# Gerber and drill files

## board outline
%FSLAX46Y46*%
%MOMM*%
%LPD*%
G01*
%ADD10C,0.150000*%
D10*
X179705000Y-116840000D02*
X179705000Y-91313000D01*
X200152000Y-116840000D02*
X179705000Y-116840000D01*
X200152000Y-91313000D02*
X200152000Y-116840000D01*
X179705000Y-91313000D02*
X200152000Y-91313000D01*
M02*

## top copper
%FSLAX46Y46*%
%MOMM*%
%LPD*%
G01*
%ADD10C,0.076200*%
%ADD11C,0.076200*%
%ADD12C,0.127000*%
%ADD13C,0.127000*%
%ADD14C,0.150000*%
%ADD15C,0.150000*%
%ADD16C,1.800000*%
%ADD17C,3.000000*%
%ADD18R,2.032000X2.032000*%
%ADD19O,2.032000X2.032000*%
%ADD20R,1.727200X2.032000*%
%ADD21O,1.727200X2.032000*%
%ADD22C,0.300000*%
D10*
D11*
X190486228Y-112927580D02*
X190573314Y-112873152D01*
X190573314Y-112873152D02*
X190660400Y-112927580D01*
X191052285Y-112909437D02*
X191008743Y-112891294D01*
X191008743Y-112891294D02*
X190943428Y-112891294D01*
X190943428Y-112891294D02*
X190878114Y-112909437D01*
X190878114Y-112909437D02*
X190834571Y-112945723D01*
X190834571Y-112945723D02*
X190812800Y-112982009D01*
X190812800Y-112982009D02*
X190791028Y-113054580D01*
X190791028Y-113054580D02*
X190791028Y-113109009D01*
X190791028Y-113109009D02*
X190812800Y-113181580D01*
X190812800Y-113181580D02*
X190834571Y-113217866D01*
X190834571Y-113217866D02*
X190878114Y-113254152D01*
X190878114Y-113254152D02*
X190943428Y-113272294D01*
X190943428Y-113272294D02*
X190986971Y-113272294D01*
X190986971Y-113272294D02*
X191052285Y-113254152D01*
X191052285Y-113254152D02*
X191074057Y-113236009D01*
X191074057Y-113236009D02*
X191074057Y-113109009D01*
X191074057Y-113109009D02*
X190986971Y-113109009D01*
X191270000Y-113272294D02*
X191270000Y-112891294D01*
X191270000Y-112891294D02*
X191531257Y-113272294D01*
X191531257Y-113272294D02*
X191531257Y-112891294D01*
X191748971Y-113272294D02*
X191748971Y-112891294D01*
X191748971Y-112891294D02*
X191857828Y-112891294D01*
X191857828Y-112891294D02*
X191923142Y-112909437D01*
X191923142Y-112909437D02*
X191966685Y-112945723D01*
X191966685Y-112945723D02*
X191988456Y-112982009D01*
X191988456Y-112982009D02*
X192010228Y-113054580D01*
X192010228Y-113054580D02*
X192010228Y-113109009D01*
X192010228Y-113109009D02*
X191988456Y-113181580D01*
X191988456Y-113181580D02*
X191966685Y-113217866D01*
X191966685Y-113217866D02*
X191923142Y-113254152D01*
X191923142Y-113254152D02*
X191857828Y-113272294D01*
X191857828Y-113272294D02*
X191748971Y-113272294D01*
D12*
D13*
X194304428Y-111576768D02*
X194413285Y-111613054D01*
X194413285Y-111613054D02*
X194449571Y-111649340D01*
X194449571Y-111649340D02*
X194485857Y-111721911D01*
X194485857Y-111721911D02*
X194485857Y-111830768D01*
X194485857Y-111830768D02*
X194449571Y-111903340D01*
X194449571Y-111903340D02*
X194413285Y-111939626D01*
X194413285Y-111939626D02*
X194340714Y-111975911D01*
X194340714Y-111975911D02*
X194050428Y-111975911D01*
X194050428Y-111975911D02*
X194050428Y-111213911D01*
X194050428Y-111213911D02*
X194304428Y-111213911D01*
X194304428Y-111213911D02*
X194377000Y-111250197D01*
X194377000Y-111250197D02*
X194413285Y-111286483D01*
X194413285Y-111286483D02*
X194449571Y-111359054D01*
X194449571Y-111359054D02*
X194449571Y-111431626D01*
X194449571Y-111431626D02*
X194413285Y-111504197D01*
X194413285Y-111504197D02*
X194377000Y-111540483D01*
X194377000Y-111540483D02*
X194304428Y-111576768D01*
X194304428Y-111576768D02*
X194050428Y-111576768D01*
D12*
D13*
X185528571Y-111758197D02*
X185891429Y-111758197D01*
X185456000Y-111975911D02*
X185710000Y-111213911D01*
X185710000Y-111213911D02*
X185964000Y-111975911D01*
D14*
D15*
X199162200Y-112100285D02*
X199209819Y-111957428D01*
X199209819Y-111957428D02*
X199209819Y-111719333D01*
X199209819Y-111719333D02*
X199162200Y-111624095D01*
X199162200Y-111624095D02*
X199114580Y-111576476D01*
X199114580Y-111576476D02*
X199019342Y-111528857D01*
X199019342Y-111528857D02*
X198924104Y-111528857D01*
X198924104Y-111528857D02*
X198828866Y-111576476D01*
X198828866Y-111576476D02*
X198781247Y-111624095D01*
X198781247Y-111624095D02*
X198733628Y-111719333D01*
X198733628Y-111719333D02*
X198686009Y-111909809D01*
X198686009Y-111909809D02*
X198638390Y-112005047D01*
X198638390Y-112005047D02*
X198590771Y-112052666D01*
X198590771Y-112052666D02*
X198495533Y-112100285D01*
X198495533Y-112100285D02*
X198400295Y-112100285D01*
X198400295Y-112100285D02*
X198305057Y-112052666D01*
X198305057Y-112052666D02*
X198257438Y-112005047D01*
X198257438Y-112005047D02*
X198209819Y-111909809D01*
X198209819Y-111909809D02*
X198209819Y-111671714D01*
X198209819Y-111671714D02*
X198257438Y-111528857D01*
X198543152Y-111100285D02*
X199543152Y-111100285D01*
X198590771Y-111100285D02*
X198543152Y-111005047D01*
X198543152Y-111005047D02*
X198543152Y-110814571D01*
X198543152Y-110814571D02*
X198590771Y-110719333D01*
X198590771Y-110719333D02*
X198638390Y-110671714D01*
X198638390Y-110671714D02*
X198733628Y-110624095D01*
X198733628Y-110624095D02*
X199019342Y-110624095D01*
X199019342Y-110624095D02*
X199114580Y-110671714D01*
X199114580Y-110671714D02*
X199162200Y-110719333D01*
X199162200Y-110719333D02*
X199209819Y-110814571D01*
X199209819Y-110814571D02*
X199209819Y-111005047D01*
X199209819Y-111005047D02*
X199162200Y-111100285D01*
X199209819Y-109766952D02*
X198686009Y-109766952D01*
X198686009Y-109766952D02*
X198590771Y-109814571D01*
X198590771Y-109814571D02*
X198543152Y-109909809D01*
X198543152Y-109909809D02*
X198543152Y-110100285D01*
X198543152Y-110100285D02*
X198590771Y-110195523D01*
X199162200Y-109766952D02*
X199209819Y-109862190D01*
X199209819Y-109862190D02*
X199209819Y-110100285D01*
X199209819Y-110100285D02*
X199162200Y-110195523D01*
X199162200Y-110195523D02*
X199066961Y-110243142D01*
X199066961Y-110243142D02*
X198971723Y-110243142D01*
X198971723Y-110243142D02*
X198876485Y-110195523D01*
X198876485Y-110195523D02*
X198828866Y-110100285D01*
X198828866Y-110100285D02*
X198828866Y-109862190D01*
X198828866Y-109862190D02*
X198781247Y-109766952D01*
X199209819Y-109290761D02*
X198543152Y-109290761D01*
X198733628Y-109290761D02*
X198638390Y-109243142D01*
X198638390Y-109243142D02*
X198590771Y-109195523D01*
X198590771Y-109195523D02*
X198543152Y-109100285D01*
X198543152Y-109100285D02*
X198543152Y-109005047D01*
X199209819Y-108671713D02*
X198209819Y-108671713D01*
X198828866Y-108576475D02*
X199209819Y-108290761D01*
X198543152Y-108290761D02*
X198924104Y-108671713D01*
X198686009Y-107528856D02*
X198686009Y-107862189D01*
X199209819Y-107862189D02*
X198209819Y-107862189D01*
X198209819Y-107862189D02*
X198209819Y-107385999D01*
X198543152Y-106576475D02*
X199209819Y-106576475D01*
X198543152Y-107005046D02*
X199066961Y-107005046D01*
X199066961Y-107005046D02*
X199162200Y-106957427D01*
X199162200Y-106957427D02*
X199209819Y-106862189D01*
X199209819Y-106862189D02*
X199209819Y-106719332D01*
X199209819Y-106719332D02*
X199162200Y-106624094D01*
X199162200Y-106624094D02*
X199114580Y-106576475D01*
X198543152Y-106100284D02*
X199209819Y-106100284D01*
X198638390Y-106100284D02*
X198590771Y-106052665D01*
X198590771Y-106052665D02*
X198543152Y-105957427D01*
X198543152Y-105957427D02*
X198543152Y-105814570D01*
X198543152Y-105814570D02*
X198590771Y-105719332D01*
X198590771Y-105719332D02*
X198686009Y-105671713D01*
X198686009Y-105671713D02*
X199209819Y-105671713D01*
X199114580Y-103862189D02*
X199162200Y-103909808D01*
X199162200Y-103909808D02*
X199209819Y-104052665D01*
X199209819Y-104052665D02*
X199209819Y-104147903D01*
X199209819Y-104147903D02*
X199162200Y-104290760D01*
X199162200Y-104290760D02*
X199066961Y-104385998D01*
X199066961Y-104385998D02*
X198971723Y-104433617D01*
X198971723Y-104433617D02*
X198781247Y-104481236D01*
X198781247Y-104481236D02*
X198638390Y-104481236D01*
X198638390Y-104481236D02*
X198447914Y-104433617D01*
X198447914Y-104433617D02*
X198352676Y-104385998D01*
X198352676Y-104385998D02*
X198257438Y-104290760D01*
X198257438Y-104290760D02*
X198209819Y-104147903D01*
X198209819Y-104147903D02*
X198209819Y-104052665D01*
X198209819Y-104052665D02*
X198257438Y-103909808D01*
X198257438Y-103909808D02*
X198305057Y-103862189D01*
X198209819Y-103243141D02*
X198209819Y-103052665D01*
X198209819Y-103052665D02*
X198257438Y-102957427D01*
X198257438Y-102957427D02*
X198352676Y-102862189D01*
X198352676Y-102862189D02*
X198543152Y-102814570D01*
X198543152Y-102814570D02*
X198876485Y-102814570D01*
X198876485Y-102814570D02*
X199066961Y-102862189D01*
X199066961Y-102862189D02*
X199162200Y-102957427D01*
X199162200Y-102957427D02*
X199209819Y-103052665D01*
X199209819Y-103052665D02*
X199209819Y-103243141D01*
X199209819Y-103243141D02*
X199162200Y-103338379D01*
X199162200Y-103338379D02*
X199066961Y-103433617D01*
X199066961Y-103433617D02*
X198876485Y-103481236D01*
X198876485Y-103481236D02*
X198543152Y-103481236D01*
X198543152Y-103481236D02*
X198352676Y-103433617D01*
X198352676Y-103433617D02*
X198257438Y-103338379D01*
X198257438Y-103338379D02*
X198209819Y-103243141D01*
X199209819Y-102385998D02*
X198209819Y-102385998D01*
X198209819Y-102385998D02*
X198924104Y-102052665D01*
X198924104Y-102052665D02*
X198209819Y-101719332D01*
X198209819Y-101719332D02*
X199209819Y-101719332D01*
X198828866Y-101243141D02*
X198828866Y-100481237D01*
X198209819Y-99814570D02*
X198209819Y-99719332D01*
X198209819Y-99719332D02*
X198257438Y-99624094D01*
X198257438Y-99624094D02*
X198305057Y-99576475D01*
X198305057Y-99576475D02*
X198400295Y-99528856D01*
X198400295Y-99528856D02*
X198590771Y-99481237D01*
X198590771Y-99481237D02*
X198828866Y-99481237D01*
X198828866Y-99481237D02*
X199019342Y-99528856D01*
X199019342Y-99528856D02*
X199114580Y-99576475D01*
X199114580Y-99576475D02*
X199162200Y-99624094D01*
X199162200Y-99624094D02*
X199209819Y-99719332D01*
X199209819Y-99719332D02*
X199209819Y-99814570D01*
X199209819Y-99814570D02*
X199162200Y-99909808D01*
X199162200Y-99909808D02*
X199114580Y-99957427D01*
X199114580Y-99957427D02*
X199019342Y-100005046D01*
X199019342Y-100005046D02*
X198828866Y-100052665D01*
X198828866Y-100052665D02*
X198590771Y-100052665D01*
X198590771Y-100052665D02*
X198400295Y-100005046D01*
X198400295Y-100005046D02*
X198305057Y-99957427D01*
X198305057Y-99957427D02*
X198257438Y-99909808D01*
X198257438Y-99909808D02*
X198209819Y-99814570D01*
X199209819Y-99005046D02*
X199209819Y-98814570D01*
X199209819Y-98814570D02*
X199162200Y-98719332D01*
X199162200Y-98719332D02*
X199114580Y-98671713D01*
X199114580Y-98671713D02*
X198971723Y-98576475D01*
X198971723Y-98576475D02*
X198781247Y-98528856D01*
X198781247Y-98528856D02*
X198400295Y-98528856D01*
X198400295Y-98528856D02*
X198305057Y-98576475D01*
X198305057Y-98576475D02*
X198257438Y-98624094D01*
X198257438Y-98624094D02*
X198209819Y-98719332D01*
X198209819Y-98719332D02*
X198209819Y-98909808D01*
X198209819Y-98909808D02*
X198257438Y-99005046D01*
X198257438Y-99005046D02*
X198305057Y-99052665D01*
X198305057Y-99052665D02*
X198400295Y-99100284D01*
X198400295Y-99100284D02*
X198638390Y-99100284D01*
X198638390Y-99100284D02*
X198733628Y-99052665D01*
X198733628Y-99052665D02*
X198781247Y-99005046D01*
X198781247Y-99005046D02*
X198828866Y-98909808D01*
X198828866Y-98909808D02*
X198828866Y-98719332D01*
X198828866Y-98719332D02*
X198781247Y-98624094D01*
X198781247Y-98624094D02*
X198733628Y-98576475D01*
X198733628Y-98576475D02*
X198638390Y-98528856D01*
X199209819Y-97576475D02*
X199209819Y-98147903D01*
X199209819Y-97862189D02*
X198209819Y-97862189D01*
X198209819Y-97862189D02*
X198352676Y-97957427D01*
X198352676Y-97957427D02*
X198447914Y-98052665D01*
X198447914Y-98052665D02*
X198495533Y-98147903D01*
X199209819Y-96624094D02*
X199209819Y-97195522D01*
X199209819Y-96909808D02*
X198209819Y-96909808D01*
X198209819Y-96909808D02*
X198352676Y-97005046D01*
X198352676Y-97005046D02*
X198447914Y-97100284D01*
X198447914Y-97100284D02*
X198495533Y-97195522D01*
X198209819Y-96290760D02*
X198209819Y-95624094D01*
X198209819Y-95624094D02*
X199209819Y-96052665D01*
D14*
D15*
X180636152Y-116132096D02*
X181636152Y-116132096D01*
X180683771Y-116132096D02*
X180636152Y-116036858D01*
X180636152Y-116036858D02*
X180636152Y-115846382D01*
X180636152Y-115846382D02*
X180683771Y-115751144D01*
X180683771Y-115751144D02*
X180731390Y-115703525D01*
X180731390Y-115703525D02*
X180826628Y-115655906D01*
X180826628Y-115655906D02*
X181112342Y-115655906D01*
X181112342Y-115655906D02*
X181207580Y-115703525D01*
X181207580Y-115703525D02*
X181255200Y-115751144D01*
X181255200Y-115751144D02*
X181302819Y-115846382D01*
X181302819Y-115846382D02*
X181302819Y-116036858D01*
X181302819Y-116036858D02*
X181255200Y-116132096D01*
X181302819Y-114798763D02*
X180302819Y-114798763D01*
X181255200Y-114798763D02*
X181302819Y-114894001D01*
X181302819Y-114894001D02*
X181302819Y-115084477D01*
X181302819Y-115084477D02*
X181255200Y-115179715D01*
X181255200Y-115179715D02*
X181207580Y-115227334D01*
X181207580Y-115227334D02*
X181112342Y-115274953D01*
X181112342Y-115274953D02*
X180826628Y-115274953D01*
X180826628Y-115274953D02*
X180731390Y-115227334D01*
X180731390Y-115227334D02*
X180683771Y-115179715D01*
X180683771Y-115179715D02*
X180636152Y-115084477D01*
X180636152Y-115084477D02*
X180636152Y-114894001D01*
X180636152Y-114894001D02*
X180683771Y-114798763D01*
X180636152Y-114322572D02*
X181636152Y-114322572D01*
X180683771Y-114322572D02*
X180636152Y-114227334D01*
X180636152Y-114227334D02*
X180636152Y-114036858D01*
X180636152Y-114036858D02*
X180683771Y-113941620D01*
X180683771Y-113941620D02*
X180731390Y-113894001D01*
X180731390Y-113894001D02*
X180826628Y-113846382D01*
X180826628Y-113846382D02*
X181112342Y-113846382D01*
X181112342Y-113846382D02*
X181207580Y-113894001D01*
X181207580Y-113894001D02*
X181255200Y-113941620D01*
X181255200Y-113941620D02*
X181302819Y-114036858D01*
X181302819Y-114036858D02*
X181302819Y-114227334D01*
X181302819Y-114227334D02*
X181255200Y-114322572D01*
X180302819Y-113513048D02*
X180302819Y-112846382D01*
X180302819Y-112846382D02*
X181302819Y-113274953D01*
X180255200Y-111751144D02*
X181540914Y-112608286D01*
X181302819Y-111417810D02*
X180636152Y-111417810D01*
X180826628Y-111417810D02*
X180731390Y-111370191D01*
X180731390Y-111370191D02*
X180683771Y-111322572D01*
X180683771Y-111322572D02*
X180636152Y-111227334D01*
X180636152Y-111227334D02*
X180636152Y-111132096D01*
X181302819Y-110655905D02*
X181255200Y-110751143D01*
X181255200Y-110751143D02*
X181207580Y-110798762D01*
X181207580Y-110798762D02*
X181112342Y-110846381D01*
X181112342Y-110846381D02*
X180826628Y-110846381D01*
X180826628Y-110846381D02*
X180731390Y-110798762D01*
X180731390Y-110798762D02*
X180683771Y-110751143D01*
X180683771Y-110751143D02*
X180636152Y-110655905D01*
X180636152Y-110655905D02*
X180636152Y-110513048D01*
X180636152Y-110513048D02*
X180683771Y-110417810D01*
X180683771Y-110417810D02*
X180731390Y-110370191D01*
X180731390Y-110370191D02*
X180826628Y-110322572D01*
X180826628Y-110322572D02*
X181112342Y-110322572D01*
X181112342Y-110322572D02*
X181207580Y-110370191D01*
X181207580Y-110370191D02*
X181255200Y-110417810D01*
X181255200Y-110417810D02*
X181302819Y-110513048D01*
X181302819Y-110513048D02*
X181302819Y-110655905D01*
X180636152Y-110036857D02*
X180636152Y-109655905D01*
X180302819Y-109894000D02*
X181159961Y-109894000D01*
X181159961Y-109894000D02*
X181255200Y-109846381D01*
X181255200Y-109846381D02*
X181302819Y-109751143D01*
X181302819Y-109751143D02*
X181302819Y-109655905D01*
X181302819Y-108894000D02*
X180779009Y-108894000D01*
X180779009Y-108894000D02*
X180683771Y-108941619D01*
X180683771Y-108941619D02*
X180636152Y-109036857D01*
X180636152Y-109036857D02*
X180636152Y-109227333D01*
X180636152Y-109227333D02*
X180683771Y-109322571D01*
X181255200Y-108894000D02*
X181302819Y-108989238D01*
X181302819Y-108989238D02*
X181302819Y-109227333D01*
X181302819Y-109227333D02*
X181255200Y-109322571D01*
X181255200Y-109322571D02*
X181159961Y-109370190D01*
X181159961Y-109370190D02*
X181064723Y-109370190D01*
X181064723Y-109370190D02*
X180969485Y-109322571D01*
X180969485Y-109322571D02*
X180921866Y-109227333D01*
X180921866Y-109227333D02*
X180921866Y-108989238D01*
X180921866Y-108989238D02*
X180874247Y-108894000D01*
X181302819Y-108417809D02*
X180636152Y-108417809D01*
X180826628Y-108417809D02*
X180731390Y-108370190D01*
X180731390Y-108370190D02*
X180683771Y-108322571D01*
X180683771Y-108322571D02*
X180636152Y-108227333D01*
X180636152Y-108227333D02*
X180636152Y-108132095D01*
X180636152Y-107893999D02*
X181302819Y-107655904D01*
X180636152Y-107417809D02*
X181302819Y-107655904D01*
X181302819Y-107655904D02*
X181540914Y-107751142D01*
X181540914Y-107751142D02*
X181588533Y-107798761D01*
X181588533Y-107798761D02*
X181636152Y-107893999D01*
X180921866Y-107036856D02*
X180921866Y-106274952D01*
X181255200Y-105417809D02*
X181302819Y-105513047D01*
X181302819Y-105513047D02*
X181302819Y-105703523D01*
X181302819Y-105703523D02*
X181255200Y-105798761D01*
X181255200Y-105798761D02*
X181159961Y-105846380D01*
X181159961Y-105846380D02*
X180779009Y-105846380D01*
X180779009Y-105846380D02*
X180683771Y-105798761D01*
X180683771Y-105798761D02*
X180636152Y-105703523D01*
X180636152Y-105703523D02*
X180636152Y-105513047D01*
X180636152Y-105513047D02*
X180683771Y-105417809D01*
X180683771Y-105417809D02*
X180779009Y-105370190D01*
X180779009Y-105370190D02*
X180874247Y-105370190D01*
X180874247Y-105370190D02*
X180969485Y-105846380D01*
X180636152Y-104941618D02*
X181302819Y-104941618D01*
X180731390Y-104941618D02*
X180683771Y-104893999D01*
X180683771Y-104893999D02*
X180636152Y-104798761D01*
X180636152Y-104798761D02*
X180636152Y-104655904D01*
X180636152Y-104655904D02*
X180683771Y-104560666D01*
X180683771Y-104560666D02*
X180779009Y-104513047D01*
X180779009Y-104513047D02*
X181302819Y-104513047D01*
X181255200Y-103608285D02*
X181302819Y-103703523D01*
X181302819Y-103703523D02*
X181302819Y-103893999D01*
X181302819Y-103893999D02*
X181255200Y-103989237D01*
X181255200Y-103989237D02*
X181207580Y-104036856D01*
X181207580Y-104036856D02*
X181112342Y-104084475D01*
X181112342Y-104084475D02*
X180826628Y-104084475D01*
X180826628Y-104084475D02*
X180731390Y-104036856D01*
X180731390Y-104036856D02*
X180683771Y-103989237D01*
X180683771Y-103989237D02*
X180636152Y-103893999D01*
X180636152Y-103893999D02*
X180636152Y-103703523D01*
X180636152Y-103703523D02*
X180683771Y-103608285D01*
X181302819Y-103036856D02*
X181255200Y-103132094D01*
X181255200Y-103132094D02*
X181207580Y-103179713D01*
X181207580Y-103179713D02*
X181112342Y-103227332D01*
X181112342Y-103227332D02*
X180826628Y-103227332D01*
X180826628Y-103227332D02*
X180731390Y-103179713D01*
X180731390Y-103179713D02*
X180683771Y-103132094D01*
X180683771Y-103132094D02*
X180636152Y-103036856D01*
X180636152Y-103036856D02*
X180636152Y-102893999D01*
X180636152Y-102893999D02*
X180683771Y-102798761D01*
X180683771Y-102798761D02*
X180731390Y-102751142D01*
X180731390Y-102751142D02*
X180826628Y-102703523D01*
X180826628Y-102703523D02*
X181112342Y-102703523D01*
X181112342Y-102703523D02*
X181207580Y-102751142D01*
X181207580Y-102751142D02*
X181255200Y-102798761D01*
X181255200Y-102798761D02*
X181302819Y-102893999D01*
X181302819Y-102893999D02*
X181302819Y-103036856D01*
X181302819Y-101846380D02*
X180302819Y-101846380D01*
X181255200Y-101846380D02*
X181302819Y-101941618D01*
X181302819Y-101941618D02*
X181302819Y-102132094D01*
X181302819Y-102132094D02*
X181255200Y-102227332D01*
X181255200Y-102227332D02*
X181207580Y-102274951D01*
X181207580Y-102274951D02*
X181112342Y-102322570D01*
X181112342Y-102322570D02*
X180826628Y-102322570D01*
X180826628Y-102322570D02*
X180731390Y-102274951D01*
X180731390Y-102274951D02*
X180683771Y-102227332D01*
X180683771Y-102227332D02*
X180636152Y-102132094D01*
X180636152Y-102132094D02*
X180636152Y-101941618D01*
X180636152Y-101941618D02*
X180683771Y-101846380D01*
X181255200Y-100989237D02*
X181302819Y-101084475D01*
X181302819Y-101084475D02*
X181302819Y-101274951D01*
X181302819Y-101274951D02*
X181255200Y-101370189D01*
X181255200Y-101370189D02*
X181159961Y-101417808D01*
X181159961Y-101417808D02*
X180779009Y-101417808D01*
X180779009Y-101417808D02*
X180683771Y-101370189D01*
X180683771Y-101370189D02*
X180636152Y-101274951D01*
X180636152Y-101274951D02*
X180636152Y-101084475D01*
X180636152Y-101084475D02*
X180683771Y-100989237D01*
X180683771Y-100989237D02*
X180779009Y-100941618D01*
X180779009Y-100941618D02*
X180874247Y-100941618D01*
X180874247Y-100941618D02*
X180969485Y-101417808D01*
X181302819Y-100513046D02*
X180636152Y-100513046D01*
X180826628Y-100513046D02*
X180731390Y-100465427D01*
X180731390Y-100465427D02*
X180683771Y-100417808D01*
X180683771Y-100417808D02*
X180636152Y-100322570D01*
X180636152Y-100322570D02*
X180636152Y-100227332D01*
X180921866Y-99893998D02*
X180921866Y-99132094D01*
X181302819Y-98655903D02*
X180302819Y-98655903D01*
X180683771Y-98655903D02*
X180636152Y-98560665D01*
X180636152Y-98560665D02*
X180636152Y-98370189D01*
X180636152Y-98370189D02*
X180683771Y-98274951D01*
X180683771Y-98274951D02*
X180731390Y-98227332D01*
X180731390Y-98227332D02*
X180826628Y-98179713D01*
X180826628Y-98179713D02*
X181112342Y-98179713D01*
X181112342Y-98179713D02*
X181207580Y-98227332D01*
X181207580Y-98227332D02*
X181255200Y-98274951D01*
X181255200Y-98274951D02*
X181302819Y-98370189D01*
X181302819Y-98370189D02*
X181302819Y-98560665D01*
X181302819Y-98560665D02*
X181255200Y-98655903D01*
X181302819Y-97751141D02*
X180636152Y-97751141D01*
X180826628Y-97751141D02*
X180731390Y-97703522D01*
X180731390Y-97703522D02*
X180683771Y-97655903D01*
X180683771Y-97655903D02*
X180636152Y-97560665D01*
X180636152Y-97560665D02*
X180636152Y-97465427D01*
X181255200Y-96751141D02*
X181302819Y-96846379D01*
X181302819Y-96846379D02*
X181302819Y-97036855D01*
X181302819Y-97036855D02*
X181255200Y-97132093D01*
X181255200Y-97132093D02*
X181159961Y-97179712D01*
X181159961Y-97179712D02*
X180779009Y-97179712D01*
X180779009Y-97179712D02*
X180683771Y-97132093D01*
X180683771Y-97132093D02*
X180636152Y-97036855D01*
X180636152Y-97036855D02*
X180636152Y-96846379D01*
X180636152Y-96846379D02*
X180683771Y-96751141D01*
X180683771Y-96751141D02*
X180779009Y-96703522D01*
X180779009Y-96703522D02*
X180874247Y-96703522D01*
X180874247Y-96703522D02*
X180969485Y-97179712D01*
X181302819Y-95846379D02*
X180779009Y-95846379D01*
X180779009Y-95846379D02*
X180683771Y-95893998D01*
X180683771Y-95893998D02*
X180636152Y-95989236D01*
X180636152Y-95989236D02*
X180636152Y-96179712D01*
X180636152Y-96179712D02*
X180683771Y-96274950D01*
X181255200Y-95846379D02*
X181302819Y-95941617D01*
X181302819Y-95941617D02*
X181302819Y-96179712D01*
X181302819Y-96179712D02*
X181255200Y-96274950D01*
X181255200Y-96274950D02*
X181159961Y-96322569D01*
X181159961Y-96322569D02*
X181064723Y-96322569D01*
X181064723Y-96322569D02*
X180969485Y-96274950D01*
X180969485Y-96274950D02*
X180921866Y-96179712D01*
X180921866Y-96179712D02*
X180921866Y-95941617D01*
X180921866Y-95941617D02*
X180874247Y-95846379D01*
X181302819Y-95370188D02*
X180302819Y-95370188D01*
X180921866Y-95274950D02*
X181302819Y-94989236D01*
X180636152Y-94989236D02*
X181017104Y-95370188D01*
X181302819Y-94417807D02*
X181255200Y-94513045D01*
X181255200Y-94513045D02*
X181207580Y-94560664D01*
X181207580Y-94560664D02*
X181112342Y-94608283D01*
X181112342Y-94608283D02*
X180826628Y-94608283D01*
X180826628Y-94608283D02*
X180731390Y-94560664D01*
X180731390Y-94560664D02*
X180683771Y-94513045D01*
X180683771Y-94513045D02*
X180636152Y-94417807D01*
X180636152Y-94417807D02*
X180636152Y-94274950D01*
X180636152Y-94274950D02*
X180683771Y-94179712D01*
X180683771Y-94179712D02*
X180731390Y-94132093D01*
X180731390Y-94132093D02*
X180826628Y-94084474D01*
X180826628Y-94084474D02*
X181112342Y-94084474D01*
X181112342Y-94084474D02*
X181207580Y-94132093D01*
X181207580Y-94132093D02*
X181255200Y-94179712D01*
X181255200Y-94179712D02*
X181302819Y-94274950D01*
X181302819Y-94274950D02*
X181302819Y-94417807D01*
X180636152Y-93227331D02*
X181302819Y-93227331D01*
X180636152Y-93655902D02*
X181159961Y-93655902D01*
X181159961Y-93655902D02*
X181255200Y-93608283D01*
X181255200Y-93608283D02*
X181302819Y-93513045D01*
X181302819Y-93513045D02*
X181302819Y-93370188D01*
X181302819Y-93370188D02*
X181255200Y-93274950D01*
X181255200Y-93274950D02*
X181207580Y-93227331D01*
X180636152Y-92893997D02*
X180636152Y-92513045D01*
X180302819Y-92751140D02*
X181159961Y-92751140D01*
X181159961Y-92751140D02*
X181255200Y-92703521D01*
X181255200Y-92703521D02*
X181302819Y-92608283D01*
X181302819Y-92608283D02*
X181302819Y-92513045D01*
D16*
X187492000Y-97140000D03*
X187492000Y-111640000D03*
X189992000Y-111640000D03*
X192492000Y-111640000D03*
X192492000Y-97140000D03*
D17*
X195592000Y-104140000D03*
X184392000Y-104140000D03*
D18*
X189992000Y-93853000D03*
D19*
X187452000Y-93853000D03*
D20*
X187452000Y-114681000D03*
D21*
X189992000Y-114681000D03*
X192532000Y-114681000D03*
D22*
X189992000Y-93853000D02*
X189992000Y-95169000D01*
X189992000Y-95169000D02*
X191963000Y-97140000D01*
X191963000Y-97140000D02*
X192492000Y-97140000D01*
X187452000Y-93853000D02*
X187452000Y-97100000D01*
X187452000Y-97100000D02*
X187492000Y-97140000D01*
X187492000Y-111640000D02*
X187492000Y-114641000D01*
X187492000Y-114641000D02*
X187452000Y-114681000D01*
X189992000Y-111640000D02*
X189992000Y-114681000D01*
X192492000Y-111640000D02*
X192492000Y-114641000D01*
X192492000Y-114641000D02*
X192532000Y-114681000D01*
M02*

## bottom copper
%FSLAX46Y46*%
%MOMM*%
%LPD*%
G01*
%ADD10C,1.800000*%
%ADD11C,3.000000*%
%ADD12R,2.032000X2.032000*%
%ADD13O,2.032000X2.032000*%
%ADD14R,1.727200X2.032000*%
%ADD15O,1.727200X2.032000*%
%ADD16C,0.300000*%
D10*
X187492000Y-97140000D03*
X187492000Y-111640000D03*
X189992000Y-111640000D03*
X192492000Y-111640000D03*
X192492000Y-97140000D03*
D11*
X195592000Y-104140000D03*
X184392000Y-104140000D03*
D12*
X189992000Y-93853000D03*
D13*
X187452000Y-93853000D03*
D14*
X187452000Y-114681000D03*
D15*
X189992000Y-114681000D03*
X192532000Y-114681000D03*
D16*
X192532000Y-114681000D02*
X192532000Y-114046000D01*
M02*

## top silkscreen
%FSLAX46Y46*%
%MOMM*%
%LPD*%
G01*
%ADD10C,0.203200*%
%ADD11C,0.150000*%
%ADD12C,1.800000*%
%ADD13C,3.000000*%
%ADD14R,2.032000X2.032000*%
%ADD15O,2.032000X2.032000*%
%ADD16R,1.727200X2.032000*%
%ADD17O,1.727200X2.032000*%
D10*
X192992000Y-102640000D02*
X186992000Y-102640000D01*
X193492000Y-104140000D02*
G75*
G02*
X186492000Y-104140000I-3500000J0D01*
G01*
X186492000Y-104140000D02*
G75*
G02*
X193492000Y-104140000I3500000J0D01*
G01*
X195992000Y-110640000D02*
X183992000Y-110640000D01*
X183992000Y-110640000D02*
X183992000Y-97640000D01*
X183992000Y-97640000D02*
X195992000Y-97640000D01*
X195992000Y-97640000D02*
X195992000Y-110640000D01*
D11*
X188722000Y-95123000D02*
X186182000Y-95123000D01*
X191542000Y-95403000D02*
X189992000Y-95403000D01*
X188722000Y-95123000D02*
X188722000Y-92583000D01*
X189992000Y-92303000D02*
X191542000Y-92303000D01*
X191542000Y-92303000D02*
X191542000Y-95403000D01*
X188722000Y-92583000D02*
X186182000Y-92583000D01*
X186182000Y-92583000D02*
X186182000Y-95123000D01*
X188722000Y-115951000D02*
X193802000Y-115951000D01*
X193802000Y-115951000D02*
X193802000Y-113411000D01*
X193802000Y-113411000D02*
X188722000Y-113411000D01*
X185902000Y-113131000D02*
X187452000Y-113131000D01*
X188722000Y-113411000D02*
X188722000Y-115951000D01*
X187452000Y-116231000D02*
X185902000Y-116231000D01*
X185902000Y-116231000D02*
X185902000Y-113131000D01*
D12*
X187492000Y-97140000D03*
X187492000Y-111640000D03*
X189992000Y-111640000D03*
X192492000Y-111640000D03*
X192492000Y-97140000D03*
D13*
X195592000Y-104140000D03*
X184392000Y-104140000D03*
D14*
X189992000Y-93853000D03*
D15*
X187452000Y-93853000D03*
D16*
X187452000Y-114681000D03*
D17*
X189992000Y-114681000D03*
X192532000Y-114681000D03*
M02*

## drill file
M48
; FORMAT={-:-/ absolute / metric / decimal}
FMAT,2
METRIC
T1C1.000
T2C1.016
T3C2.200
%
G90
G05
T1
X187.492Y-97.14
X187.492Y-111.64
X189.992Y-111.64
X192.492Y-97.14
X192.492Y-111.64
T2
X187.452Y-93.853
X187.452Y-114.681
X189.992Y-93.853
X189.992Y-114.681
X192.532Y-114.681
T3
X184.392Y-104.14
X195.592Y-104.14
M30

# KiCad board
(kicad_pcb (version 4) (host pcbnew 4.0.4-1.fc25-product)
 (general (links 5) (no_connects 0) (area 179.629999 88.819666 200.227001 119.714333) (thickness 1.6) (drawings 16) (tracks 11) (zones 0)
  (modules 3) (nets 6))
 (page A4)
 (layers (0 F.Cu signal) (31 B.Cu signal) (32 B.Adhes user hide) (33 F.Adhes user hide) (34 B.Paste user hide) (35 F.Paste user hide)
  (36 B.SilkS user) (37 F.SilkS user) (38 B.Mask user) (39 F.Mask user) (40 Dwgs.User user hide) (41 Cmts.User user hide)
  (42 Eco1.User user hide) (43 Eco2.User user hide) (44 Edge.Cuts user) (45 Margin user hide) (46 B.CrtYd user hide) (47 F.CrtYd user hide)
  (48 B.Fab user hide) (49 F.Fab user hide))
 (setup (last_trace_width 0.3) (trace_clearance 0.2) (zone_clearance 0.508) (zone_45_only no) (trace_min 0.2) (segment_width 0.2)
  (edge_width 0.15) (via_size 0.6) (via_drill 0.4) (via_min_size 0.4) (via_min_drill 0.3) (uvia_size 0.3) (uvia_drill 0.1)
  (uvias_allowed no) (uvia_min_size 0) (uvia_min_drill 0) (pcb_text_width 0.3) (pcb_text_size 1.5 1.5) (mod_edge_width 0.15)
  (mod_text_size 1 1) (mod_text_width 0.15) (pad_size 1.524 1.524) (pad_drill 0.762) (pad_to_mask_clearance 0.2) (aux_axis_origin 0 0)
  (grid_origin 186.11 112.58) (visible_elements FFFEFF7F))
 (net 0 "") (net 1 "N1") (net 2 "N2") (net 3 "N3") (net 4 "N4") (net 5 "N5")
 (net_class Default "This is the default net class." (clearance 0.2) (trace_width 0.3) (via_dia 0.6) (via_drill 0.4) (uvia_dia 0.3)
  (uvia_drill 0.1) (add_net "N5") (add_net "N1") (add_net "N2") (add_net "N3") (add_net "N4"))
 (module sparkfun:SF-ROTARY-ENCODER (layer F.Cu) (at 189.992 104.14)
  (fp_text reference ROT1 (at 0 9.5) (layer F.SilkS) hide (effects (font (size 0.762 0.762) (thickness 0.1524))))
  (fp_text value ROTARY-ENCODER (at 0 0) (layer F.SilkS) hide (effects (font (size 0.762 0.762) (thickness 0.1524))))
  (fp_line (start 3 -1.5) (end -3 -1.5) (layer F.SilkS) (width 0.2032))
  (fp_circle (center 0 0) (end 3.5 0) (layer F.SilkS) (width 0.2032))
  (fp_line (start 6 6.5) (end -6 6.5) (layer F.SilkS) (width 0.2032))
  (fp_line (start -6 6.5) (end -6 -6.5) (layer F.SilkS) (width 0.2032))
  (fp_line (start -6 -6.5) (end 6 -6.5) (layer F.SilkS) (width 0.2032))
  (fp_line (start 6 -6.5) (end 6 6.5) (layer F.SilkS) (width 0.2032))
  (pad 1 thru_hole circle (at -2.5 -7) (size 1.8 1.8) (drill 1) (layers *.Cu *.Mask F.SilkS) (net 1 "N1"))
  (pad 2 thru_hole circle (at -2.5 7.5) (size 1.8 1.8) (drill 1) (layers *.Cu *.Mask F.SilkS) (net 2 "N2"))
  (pad 3 thru_hole circle (at 0 7.5) (size 1.8 1.8) (drill 1) (layers *.Cu *.Mask F.SilkS) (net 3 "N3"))
  (pad 4 thru_hole circle (at 2.5 7.5) (size 1.8 1.8) (drill 1) (layers *.Cu *.Mask F.SilkS) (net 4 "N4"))
  (pad 5 thru_hole circle (at 2.5 -7) (size 1.8 1.8) (drill 1) (layers *.Cu *.Mask F.SilkS) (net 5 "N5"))
  (pad "" thru_hole circle (at 5.6 0) (size 3 3) (drill 2.2) (layers *.Cu *.Mask F.SilkS))
  (pad "" thru_hole circle (at -5.6 0) (size 3 3) (drill 2.2) (layers *.Cu *.Mask F.SilkS)))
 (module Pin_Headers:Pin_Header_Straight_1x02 (layer F.Cu) (at 189.992 93.853 270)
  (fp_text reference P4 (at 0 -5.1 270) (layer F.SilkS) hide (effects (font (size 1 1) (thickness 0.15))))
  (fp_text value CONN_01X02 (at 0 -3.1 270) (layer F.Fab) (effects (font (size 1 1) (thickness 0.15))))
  (fp_line (start 1.27 1.27) (end 1.27 3.81) (layer F.SilkS) (width 0.15))
  (fp_line (start 1.55 -1.55) (end 1.55 0) (layer F.SilkS) (width 0.15))
  (fp_line (start 1.27 1.27) (end -1.27 1.27) (layer F.SilkS) (width 0.15))
  (fp_line (start -1.55 0) (end -1.55 -1.55) (layer F.SilkS) (width 0.15))
  (fp_line (start -1.55 -1.55) (end 1.55 -1.55) (layer F.SilkS) (width 0.15))
  (fp_line (start -1.27 1.27) (end -1.27 3.81) (layer F.SilkS) (width 0.15))
  (fp_line (start -1.27 3.81) (end 1.27 3.81) (layer F.SilkS) (width 0.15))
  (pad 1 thru_hole rect (at 0 0 270) (size 2.032 2.032) (drill 1.016) (layers *.Cu *.Mask F.SilkS) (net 5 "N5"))
  (pad 2 thru_hole oval (at 0 2.54 270) (size 2.032 2.032) (drill 1.016) (layers *.Cu *.Mask F.SilkS) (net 1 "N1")))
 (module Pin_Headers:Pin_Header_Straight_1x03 (layer F.Cu) (at 187.452 114.681 90)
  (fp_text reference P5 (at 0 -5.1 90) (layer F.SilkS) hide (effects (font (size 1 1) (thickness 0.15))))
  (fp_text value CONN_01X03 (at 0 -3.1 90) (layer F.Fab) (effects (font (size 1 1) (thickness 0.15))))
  (fp_line (start -1.27 1.27) (end -1.27 6.35) (layer F.SilkS) (width 0.15))
  (fp_line (start -1.27 6.35) (end 1.27 6.35) (layer F.SilkS) (width 0.15))
  (fp_line (start 1.27 6.35) (end 1.27 1.27) (layer F.SilkS) (width 0.15))
  (fp_line (start 1.55 -1.55) (end 1.55 0) (layer F.SilkS) (width 0.15))
  (fp_line (start 1.27 1.27) (end -1.27 1.27) (layer F.SilkS) (width 0.15))
  (fp_line (start -1.55 0) (end -1.55 -1.55) (layer F.SilkS) (width 0.15))
  (fp_line (start -1.55 -1.55) (end 1.55 -1.55) (layer F.SilkS) (width 0.15))
  (pad 1 thru_hole rect (at 0 0 90) (size 2.032 1.7272) (drill 1.016) (layers *.Cu *.Mask F.SilkS) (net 2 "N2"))
  (pad 2 thru_hole oval (at 0 2.54 90) (size 2.032 1.7272) (drill 1.016) (layers *.Cu *.Mask F.SilkS) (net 3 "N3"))
  (pad 3 thru_hole oval (at 0 5.08 90) (size 2.032 1.7272) (drill 1.016) (layers *.Cu *.Mask F.SilkS) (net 4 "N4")))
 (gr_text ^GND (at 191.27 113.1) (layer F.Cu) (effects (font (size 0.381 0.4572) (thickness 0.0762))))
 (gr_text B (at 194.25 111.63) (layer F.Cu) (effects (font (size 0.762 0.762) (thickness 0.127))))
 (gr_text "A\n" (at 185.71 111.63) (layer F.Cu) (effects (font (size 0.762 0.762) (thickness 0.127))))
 (gr_line (start 179.705 116.84) (end 179.705 91.313) (angle 90) (layer Edge.Cuts) (width 0.15))
 (gr_line (start 200.152 116.84) (end 179.705 116.84) (angle 90) (layer Edge.Cuts) (width 0.15))
 (gr_line (start 200.152 91.313) (end 200.152 116.84) (angle 90) (layer Edge.Cuts) (width 0.15))
 (gr_line (start 179.705 91.313) (end 200.152 91.313) (angle 90) (layer Edge.Cuts) (width 0.15))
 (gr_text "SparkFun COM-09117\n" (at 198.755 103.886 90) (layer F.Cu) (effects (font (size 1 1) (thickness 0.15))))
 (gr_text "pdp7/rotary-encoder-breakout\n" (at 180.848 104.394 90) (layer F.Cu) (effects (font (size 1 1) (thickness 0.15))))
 (segment (start 189.992 93.853) (end 189.992 95.169) (width 0.3) (layer F.Cu) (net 5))
 (segment (start 189.992 95.169) (end 191.963 97.14) (width 0.3) (layer F.Cu) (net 5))
 (segment (start 191.963 97.14) (end 192.492 97.14) (width 0.3) (layer F.Cu) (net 5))
 (segment (start 187.452 93.853) (end 187.452 97.1) (width 0.3) (layer F.Cu) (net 1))
 (segment (start 187.452 97.1) (end 187.492 97.14) (width 0.3) (layer F.Cu) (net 1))
 (segment (start 187.492 111.64) (end 187.492 114.641) (width 0.3) (layer F.Cu) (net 2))
 (segment (start 187.492 114.641) (end 187.452 114.681) (width 0.3) (layer F.Cu) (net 2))
 (segment (start 189.992 111.64) (end 189.992 114.681) (width 0.3) (layer F.Cu) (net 3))
 (segment (start 192.492 111.64) (end 192.492 114.641) (width 0.3) (layer F.Cu) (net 4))
 (segment (start 192.492 114.641) (end 192.532 114.681) (width 0.3) (layer F.Cu) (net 4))
 (segment (start 192.532 114.681) (end 192.532 114.046) (width 0.3) (layer B.Cu) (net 4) (status 80000)))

